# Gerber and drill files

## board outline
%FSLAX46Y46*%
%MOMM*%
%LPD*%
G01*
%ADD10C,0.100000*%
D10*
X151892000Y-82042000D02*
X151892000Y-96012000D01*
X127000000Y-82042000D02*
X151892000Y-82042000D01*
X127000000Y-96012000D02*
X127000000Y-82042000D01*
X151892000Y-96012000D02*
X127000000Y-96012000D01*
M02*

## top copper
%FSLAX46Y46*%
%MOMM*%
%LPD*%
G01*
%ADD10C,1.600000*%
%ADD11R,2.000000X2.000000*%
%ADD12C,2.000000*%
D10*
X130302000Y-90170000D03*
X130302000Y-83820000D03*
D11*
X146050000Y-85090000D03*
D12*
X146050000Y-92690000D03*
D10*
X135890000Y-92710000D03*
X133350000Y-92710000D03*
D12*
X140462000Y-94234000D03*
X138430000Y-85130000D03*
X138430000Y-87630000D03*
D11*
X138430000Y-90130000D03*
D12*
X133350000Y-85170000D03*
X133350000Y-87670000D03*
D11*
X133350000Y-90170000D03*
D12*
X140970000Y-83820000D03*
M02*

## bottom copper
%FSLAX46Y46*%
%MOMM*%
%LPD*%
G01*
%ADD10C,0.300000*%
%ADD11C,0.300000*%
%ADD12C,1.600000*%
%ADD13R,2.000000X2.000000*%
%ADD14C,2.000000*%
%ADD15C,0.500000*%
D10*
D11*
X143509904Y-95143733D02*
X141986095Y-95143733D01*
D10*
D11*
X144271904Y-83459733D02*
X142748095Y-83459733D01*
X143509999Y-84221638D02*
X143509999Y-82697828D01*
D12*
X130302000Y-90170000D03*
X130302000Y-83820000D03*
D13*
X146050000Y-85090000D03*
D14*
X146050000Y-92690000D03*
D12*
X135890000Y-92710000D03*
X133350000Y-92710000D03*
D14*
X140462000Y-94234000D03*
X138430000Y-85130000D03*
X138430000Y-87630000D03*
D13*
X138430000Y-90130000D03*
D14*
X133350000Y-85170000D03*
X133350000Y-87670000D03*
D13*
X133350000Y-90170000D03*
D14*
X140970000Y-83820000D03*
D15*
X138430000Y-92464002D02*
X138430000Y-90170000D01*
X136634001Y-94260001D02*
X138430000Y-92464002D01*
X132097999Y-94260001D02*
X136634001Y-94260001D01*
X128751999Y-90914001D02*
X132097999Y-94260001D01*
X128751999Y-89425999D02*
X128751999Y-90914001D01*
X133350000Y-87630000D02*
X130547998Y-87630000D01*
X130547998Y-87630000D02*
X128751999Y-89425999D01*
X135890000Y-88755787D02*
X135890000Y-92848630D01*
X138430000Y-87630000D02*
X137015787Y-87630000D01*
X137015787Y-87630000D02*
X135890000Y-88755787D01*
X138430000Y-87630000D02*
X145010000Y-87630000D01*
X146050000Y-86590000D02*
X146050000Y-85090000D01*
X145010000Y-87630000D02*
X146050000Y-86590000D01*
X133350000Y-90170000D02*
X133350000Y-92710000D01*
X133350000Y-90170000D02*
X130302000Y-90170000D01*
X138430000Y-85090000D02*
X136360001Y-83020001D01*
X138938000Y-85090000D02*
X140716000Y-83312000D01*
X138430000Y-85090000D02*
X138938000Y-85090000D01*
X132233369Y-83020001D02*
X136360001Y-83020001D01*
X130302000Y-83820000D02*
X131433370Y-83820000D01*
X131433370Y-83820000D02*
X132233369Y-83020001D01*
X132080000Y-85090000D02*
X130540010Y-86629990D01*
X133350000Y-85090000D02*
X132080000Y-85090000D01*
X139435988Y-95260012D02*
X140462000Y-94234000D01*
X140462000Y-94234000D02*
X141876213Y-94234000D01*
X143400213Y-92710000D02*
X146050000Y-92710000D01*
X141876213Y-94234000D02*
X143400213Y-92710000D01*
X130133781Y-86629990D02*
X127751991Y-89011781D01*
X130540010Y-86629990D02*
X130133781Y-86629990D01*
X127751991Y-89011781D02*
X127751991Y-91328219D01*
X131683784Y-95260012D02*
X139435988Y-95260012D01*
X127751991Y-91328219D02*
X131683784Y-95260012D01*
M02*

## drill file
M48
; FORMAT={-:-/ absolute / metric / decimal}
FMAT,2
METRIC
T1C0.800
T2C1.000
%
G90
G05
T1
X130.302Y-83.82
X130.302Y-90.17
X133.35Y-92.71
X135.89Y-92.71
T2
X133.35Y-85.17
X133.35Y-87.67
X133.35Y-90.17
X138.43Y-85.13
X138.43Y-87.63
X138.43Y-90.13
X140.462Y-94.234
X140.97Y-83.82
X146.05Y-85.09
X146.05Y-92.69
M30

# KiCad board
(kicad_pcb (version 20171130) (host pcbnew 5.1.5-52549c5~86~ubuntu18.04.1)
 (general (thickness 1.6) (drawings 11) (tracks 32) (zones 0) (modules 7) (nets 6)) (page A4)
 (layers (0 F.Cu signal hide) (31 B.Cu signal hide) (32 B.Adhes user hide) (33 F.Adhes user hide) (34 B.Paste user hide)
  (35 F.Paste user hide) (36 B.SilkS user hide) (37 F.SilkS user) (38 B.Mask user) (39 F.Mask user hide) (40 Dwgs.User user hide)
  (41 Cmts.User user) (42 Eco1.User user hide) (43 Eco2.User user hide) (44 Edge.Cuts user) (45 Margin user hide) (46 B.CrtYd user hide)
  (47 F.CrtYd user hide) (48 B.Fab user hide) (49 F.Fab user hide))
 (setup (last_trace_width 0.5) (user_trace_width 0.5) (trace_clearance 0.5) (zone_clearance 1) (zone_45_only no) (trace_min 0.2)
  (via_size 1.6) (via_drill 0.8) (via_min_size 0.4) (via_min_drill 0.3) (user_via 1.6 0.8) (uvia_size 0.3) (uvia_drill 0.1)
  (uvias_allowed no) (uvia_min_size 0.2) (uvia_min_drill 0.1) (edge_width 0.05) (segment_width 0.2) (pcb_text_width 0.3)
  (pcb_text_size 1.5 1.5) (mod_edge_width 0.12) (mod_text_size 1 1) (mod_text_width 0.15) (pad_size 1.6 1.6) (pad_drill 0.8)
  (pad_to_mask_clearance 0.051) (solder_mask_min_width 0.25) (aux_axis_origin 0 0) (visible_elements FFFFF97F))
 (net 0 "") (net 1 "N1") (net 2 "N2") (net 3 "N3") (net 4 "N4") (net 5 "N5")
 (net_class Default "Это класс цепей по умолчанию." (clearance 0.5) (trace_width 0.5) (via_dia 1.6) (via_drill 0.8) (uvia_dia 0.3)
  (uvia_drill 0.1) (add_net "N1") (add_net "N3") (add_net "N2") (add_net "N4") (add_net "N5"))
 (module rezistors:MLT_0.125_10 (layer F.Cu) (at 130.302 87.63 90)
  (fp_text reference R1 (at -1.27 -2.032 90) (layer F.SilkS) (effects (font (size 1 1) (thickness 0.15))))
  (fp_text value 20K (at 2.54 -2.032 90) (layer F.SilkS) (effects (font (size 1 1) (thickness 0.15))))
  (pad 1 thru_hole circle (at -2.54 0 90) (size 1.6 1.6) (drill 0.8) (layers *.Cu *.Mask F.SilkS) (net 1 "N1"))
  (pad 2 thru_hole circle (at 3.81 0 90) (size 1.6 1.6) (drill 0.8) (layers *.Cu *.Mask F.SilkS) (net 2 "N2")))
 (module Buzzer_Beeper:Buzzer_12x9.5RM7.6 (layer F.Cu) (at 146.05 85.09 270)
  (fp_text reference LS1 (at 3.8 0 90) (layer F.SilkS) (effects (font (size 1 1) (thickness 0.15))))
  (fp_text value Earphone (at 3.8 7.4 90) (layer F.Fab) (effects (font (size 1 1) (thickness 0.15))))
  (pad 1 thru_hole rect (at 0 0 270) (size 2 2) (drill 1) (layers *.Cu *.Mask) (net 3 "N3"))
  (pad 2 thru_hole circle (at 7.6 0 270) (size 2 2) (drill 1) (layers *.Cu *.Mask) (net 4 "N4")))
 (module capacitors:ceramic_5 (layer F.Cu) (at 134.62 92.71) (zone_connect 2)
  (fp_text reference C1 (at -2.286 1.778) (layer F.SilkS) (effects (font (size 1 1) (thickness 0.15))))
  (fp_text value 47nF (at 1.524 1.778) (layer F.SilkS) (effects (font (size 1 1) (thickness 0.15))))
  (pad 2 thru_hole circle (at 1.27 0) (size 1.6 1.6) (drill 0.8) (layers *.Cu *.Mask F.SilkS) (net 3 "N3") (zone_connect 2))
  (pad 1 thru_hole circle (at -1.27 0) (size 1.6 1.6) (drill 0.8) (layers *.Cu *.Mask F.SilkS) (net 1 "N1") (zone_connect 2)))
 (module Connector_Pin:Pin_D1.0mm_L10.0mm (layer F.Cu) (at 140.462 94.234)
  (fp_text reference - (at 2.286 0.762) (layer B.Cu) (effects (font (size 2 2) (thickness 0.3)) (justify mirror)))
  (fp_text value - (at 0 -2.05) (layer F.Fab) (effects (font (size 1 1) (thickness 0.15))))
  (pad 1 thru_hole circle (at 0 0) (size 2 2) (drill 1) (layers *.Cu *.Mask) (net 4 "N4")))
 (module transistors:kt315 (layer F.Cu) (at 138.43 87.63 270)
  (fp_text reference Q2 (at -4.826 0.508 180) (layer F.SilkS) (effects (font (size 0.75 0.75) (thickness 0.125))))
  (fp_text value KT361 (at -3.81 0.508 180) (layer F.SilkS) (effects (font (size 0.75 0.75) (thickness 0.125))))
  (pad E thru_hole circle (at -2.5 0 270) (size 2 2) (drill 1) (layers *.Cu *.Mask F.SilkS) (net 2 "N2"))
  (pad C thru_hole circle (at 0 0 270) (size 2 2) (drill 1) (layers *.Cu *.Mask F.SilkS) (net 3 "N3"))
  (pad B thru_hole rect (at 2.5 0 270) (size 2 2) (drill 1) (layers *.Cu *.Mask F.SilkS) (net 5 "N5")))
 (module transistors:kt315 (layer F.Cu) (at 133.35 87.67 270)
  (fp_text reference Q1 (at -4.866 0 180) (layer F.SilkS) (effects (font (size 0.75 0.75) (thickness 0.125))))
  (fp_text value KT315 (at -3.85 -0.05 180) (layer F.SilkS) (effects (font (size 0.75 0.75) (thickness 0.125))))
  (pad E thru_hole circle (at -2.5 0 270) (size 2 2) (drill 1) (layers *.Cu *.Mask F.SilkS) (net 4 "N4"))
  (pad C thru_hole circle (at 0 0 270) (size 2 2) (drill 1) (layers *.Cu *.Mask F.SilkS) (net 5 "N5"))
  (pad B thru_hole rect (at 2.5 0 270) (size 2 2) (drill 1) (layers *.Cu *.Mask F.SilkS) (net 1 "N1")))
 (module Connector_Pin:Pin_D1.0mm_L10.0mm (layer F.Cu) (at 140.97 83.82)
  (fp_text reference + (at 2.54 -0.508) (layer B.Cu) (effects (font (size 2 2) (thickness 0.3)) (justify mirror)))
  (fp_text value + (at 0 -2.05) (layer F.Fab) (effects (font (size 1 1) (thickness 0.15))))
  (pad 1 thru_hole circle (at 0 0) (size 2 2) (drill 1) (layers *.Cu *.Mask) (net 2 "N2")))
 (gr_line (start 151.892 82.042) (end 151.892 96.012) (layer Edge.Cuts) (width 0.1))
 (gr_line (start 127 82.042) (end 151.892 82.042) (layer Edge.Cuts) (width 0.1))
 (gr_line (start 127 96.012) (end 127 82.042) (layer Edge.Cuts) (width 0.1))
 (gr_line (start 151.892 96.012) (end 127 96.012) (layer Edge.Cuts) (width 0.1))
 (segment (start 138.43 92.464002) (end 138.43 90.17) (width 0.5) (layer B.Cu) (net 5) (status 20))
 (segment (start 136.634001 94.260001) (end 138.43 92.464002) (width 0.5) (layer B.Cu) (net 5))
 (segment (start 132.097999 94.260001) (end 136.634001 94.260001) (width 0.5) (layer B.Cu) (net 5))
 (segment (start 128.751999 90.914001) (end 132.097999 94.260001) (width 0.5) (layer B.Cu) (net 5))
 (segment (start 128.751999 89.425999) (end 128.751999 90.914001) (width 0.5) (layer B.Cu) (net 5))
 (segment (start 133.35 87.63) (end 130.547998 87.63) (width 0.5) (layer B.Cu) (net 5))
 (segment (start 130.547998 87.63) (end 128.751999 89.425999) (width 0.5) (layer B.Cu) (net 5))
 (segment (start 135.89 88.755787) (end 135.89 92.84863) (width 0.5) (layer B.Cu) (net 3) (status 20))
 (segment (start 138.43 87.63) (end 137.015787 87.63) (width 0.5) (layer B.Cu) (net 3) (status 10))
 (segment (start 137.015787 87.63) (end 135.89 88.755787) (width 0.5) (layer B.Cu) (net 3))
 (segment (start 138.43 87.63) (end 145.01 87.63) (width 0.5) (layer B.Cu) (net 3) (status 10))
 (segment (start 146.05 86.59) (end 146.05 85.09) (width 0.5) (layer B.Cu) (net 3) (status 20))
 (segment (start 145.01 87.63) (end 146.05 86.59) (width 0.5) (layer B.Cu) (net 3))
 (segment (start 133.35 90.17) (end 133.35 92.71) (width 0.5) (layer B.Cu) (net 1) (status 30))
 (segment (start 133.35 90.17) (end 130.302 90.17) (width 0.5) (layer B.Cu) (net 1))
 (segment (start 138.43 85.09) (end 136.360001 83.020001) (width 0.5) (layer B.Cu) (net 2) (status 10))
 (segment (start 138.938 85.09) (end 140.716 83.312) (width 0.5) (layer B.Cu) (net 2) (status 30))
 (segment (start 138.43 85.09) (end 138.938 85.09) (width 0.5) (layer B.Cu) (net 2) (status 30))
 (segment (start 132.233369 83.020001) (end 136.360001 83.020001) (width 0.5) (layer B.Cu) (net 2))
 (segment (start 130.302 83.82) (end 131.43337 83.82) (width 0.5) (layer B.Cu) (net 2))
 (segment (start 131.43337 83.82) (end 132.233369 83.020001) (width 0.5) (layer B.Cu) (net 2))
 (segment (start 132.08 85.09) (end 130.54001 86.62999) (width 0.5) (layer B.Cu) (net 4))
 (segment (start 133.35 85.09) (end 132.08 85.09) (width 0.5) (layer B.Cu) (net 4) (status 10))
 (segment (start 139.435988 95.260012) (end 140.462 94.234) (width 0.5) (layer B.Cu) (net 4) (status 20))
 (segment (start 140.462 94.234) (end 141.876213 94.234) (width 0.5) (layer B.Cu) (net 4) (status 10))
 (segment (start 143.400213 92.71) (end 146.05 92.71) (width 0.5) (layer B.Cu) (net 4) (status 20))
 (segment (start 141.876213 94.234) (end 143.400213 92.71) (width 0.5) (layer B.Cu) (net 4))
 (segment (start 130.133781 86.62999) (end 127.751991 89.011781) (width 0.5) (layer B.Cu) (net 4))
 (segment (start 130.54001 86.62999) (end 130.133781 86.62999) (width 0.5) (layer B.Cu) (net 4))
 (segment (start 127.751991 89.011781) (end 127.751991 91.328219) (width 0.5) (layer B.Cu) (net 4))
 (segment (start 131.683784 95.260012) (end 139.435988 95.260012) (width 0.5) (layer B.Cu) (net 4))
 (segment (start 127.751991 91.328219) (end 131.683784 95.260012) (width 0.5) (layer B.Cu) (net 4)))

